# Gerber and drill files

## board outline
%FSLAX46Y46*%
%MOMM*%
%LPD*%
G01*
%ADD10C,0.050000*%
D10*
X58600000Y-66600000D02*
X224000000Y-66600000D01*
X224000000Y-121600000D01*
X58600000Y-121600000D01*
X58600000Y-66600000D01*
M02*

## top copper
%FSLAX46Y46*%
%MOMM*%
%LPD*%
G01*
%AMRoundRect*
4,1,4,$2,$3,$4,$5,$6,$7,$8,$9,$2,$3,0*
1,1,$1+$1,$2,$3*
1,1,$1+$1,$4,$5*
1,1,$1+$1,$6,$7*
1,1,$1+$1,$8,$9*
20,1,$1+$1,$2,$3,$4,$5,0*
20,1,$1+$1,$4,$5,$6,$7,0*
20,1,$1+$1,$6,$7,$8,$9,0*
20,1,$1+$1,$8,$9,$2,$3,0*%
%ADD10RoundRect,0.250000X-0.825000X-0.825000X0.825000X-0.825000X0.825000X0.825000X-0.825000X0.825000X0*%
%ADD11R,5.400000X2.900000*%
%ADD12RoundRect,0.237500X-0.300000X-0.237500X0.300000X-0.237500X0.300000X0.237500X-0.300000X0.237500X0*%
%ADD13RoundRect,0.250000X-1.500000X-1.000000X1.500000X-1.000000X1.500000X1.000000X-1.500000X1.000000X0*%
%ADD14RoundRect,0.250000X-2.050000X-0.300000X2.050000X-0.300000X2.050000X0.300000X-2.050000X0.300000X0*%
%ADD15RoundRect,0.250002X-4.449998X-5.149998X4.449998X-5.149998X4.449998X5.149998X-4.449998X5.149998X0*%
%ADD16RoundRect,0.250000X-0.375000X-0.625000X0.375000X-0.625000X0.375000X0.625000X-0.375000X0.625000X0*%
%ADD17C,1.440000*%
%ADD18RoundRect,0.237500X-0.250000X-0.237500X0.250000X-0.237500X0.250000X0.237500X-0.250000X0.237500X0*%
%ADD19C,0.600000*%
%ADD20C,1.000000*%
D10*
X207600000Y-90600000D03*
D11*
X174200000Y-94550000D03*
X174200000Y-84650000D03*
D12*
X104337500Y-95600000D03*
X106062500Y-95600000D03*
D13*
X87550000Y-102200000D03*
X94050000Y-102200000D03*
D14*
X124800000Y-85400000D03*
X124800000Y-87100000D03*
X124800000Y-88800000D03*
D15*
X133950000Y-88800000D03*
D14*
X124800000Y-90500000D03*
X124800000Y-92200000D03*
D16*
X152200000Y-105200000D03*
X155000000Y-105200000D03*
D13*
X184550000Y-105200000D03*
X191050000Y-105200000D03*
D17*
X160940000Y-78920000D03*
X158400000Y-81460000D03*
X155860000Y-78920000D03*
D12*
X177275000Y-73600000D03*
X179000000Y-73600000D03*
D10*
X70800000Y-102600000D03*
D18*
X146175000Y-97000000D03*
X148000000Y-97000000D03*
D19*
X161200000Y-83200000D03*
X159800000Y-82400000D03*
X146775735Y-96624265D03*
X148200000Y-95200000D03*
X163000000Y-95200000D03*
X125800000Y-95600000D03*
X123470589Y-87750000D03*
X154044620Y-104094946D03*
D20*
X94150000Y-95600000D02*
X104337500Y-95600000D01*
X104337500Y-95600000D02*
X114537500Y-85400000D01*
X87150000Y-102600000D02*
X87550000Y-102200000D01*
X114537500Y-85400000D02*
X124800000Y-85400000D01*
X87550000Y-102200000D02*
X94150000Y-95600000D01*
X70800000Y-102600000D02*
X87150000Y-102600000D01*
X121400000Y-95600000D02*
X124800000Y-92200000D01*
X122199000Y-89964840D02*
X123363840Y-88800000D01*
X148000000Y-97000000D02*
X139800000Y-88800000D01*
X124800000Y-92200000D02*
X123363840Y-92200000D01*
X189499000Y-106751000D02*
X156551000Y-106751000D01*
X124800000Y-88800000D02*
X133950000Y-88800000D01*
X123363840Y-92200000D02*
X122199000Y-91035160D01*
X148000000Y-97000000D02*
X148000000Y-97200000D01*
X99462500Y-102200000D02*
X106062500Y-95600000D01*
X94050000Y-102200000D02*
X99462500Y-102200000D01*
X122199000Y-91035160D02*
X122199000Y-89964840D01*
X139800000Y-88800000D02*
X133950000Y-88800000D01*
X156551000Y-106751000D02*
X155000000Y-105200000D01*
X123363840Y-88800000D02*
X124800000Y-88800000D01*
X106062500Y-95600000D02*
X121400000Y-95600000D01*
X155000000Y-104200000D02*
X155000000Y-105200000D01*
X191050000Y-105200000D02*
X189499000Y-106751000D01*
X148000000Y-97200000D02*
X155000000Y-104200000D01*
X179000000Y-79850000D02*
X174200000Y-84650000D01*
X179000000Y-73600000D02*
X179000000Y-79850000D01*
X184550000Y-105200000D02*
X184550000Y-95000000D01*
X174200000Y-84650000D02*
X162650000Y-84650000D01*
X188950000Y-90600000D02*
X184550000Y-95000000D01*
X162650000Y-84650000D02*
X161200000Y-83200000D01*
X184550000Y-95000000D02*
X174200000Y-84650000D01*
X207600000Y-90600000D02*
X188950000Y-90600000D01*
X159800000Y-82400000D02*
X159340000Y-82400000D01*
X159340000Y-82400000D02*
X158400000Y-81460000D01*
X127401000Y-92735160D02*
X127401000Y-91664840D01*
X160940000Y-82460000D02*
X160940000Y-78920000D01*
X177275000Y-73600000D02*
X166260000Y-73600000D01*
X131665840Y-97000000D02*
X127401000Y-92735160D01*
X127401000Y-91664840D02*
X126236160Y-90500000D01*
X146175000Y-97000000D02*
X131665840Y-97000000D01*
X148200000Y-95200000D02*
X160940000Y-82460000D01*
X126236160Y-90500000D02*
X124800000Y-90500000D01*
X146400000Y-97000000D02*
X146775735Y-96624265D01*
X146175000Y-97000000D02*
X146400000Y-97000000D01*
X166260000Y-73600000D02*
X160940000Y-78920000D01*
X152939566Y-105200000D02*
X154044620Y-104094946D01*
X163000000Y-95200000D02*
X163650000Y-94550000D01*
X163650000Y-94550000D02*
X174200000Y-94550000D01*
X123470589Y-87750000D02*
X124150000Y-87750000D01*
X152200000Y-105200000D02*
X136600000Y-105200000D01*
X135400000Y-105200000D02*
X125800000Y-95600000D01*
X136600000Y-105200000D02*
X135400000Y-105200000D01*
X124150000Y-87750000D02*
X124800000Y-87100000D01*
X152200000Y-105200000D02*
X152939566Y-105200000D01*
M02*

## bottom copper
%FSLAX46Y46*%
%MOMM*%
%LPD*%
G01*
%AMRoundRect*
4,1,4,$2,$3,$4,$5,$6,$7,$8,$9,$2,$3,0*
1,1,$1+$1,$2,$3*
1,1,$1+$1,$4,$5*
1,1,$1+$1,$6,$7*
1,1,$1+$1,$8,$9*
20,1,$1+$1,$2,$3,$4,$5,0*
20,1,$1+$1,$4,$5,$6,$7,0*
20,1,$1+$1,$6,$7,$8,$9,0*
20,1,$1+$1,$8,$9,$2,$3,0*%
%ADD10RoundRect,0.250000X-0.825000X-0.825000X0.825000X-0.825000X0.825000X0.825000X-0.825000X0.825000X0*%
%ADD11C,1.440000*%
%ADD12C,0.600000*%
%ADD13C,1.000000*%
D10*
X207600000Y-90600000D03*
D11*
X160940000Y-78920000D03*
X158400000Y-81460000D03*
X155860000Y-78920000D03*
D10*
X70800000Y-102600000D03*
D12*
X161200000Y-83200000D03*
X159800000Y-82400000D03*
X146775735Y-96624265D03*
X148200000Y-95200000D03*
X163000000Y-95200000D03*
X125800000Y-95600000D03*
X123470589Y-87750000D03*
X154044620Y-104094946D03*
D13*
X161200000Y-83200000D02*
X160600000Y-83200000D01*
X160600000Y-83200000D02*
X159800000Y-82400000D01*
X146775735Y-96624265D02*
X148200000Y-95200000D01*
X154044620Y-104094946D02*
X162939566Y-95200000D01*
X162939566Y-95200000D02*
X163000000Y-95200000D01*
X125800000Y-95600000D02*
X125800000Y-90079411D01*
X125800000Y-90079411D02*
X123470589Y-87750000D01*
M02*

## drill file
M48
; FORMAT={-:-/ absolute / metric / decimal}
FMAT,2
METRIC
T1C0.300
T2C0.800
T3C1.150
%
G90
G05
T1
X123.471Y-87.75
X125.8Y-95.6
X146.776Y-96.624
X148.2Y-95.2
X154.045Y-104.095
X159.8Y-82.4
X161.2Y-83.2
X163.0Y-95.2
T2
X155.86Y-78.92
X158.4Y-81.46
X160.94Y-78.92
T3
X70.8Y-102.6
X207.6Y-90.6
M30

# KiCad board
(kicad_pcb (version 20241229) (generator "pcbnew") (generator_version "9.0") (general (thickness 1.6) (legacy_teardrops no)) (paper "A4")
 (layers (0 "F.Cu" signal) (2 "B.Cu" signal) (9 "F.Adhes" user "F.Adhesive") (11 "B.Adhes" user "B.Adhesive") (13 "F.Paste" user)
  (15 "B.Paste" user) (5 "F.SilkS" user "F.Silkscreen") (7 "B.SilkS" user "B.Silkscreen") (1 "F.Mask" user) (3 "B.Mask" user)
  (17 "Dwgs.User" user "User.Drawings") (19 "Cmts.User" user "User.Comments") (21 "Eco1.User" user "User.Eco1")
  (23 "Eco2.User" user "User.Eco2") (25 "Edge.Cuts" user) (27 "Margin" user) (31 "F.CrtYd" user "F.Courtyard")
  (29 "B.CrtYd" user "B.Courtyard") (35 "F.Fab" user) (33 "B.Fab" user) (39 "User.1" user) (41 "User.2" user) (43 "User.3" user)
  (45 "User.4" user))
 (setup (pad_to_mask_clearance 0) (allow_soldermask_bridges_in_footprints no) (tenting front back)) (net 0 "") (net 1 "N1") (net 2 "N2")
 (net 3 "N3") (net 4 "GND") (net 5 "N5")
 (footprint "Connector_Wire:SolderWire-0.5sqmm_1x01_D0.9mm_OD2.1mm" (layer "F.Cu") (at 207.6 90.6)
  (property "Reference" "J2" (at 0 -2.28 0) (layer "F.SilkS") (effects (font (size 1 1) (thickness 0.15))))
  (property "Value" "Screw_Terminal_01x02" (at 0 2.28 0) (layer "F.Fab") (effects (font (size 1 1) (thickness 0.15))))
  (pad "1" thru_hole roundrect (at 0 0) (size 2.15 2.15) (drill 1.15) (layers "*.Cu" "*.Mask") (remove_unused_layers no)
   (roundrect_rratio 0.116279) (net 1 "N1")))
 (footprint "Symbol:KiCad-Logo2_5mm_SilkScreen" (layer "F.Cu") (at 66.4 70.6)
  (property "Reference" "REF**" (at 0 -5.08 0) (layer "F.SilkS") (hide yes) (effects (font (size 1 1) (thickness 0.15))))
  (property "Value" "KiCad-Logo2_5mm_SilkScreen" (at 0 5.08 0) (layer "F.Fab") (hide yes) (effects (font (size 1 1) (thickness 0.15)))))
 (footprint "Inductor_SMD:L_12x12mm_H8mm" (layer "F.Cu") (at 174.2 89.6 90)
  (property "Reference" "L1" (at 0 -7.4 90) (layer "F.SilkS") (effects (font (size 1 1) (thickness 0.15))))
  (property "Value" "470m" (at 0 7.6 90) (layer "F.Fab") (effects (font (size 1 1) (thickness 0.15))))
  (pad "1" smd rect (at -4.95 0 90) (size 2.9 5.4) (layers "F.Cu" "F.Mask" "F.Paste") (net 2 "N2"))
  (pad "2" smd rect (at 4.95 0 90) (size 2.9 5.4) (layers "F.Cu" "F.Mask" "F.Paste") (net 1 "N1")))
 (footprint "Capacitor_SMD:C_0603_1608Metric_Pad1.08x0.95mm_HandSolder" (layer "F.Cu") (at 105.2 95.6)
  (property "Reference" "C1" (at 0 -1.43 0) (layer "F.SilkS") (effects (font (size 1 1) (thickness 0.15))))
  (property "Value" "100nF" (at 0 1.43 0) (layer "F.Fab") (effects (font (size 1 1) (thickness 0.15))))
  (pad "1" smd roundrect (at -0.8625 0) (size 1.075 0.95) (layers "F.Cu" "F.Mask" "F.Paste") (roundrect_rratio 0.25) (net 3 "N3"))
  (pad "2" smd roundrect (at 0.8625 0) (size 1.075 0.95) (layers "F.Cu" "F.Mask" "F.Paste") (roundrect_rratio 0.25) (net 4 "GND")))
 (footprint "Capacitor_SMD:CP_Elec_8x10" (layer "F.Cu") (at 90.8 102.2)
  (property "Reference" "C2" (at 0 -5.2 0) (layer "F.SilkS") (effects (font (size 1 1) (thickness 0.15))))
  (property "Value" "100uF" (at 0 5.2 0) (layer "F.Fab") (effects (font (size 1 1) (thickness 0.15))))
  (pad "1" smd roundrect (at -3.25 0) (size 3.5 2.5) (layers "F.Cu" "F.Mask" "F.Paste") (roundrect_rratio 0.1) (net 3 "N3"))
  (pad "2" smd roundrect (at 3.25 0) (size 3.5 2.5) (layers "F.Cu" "F.Mask" "F.Paste") (roundrect_rratio 0.1) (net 4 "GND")))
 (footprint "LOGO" (layer "F.Cu") (at 217.6 114.8)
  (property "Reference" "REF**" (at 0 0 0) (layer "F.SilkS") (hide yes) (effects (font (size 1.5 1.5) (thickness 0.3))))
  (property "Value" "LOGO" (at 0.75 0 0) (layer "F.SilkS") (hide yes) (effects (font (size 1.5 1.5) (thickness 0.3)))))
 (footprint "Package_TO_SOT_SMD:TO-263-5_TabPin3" (layer "F.Cu") (at 132.45 88.8)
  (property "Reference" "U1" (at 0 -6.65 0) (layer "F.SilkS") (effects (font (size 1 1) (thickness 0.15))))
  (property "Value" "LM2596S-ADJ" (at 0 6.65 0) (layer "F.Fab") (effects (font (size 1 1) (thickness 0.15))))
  (pad "" smd roundrect (at -0.925 -2.775) (size 4.55 5.25) (layers "F.Paste") (roundrect_rratio 0.054945))
  (pad "" smd roundrect (at -0.925 2.775) (size 4.55 5.25) (layers "F.Paste") (roundrect_rratio 0.054945))
  (pad "" smd roundrect (at 3.925 -2.775) (size 4.55 5.25) (layers "F.Paste") (roundrect_rratio 0.054945))
  (pad "" smd roundrect (at 3.925 2.775) (size 4.55 5.25) (layers "F.Paste") (roundrect_rratio 0.054945))
  (pad "1" smd roundrect (at -7.65 -3.4) (size 4.6 1.1) (layers "F.Cu" "F.Mask" "F.Paste") (roundrect_rratio 0.227273) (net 3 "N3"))
  (pad "2" smd roundrect (at -7.65 -1.7) (size 4.6 1.1) (layers "F.Cu" "F.Mask" "F.Paste") (roundrect_rratio 0.227273) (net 2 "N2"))
  (pad "3" smd roundrect (at -7.65 0) (size 4.6 1.1) (layers "F.Cu" "F.Mask" "F.Paste") (roundrect_rratio 0.227273) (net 4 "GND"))
  (pad "3" smd roundrect (at 1.5 0) (size 9.4 10.8) (layers "F.Cu" "F.Mask") (roundrect_rratio 0.026596) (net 4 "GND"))
  (pad "4" smd roundrect (at -7.65 1.7) (size 4.6 1.1) (layers "F.Cu" "F.Mask" "F.Paste") (roundrect_rratio 0.227273) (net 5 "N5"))
  (pad "5" smd roundrect (at -7.65 3.4) (size 4.6 1.1) (layers "F.Cu" "F.Mask" "F.Paste") (roundrect_rratio 0.227273) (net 4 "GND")))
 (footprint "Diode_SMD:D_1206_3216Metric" (layer "F.Cu") (at 153.6 105.2)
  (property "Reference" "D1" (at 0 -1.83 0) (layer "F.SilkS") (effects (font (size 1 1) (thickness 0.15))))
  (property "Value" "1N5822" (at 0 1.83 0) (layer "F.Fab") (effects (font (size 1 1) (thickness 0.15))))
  (pad "1" smd roundrect (at -1.4 0) (size 1.25 1.75) (layers "F.Cu" "F.Mask" "F.Paste") (roundrect_rratio 0.2) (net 2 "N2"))
  (pad "2" smd roundrect (at 1.4 0) (size 1.25 1.75) (layers "F.Cu" "F.Mask" "F.Paste") (roundrect_rratio 0.2) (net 4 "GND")))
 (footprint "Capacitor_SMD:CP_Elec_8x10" (layer "F.Cu") (at 187.8 105.2)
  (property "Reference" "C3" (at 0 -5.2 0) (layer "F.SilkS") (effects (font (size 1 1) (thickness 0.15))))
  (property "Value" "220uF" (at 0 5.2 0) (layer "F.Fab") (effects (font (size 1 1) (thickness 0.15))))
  (pad "1" smd roundrect (at -3.25 0) (size 3.5 2.5) (layers "F.Cu" "F.Mask" "F.Paste") (roundrect_rratio 0.1) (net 1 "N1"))
  (pad "2" smd roundrect (at 3.25 0) (size 3.5 2.5) (layers "F.Cu" "F.Mask" "F.Paste") (roundrect_rratio 0.1) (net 4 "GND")))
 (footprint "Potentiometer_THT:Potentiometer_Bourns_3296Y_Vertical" (layer "F.Cu") (at 160.94 78.92)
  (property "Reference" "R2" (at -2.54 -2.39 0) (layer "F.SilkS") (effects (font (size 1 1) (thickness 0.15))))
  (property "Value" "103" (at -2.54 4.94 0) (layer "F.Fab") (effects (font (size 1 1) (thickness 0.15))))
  (pad "1" thru_hole circle (at 0 0) (size 1.44 1.44) (drill 0.8) (layers "*.Cu" "*.Mask") (remove_unused_layers no) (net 5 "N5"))
  (pad "2" thru_hole circle (at -2.54 2.54) (size 1.44 1.44) (drill 0.8) (layers "*.Cu" "*.Mask") (remove_unused_layers no) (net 1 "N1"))
  (pad "3" thru_hole circle (at -5.08 0) (size 1.44 1.44) (drill 0.8) (layers "*.Cu" "*.Mask") (remove_unused_layers no)))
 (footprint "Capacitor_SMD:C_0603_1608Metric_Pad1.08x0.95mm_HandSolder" (layer "F.Cu") (at 178.1375 73.6)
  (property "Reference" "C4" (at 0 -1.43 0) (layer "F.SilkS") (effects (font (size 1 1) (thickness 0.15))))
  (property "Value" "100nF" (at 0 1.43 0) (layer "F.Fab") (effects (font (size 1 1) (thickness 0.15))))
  (pad "1" smd roundrect (at -0.8625 0) (size 1.075 0.95) (layers "F.Cu" "F.Mask" "F.Paste") (roundrect_rratio 0.25) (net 5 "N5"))
  (pad "2" smd roundrect (at 0.8625 0) (size 1.075 0.95) (layers "F.Cu" "F.Mask" "F.Paste") (roundrect_rratio 0.25) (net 1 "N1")))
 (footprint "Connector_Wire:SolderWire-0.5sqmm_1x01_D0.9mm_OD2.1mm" (layer "F.Cu") (at 70.8 102.6)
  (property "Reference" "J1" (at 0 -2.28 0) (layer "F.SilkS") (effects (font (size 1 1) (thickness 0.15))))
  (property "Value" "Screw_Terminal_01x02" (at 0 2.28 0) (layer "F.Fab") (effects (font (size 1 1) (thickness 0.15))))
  (pad "1" thru_hole roundrect (at 0 0) (size 2.15 2.15) (drill 1.15) (layers "*.Cu" "*.Mask") (remove_unused_layers no)
   (roundrect_rratio 0.116279) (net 3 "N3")))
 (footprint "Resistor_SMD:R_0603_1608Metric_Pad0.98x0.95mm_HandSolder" (layer "F.Cu") (at 147.0875 97)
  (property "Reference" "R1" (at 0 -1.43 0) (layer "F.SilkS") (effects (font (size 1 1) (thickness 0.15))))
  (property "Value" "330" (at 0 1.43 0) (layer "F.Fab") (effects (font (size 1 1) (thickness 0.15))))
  (pad "1" smd roundrect (at -0.9125 0) (size 0.975 0.95) (layers "F.Cu" "F.Mask" "F.Paste") (roundrect_rratio 0.25) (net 5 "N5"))
  (pad "2" smd roundrect (at 0.9125 0) (size 0.975 0.95) (layers "F.Cu" "F.Mask" "F.Paste") (roundrect_rratio 0.25) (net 4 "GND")))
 (gr_rect (start 58.6 66.6) (end 224 121.6) (stroke (width 0.05) (type default)) (fill no) (layer "Edge.Cuts"))
 (segment (start 94.15 95.6) (end 104.3375 95.6) (width 1) (layers "F.Cu" "F.Mask") (solder_mask_margin 1) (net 3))
 (segment (start 104.3375 95.6) (end 114.5375 85.4) (width 1) (layers "F.Cu" "F.Mask") (solder_mask_margin 1) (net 3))
 (segment (start 87.15 102.6) (end 87.55 102.2) (width 1) (layer "F.Cu") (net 3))
 (segment (start 114.5375 85.4) (end 124.8 85.4) (width 1) (layers "F.Cu" "F.Mask") (solder_mask_margin 1) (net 3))
 (segment (start 87.55 102.2) (end 94.15 95.6) (width 1) (layers "F.Cu" "F.Mask") (solder_mask_margin 1) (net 3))
 (segment (start 70.8 102.6) (end 87.15 102.6) (width 1) (layers "F.Cu" "F.Mask") (solder_mask_margin 1) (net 3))
 (segment (start 121.4 95.6) (end 124.8 92.2) (width 1) (layers "F.Cu" "F.Mask") (solder_mask_margin 1) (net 4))
 (segment (start 122.199 89.96484) (end 123.36384 88.8) (width 1) (layers "F.Cu" "F.Mask") (solder_mask_margin 1) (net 4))
 (segment (start 148 97) (end 139.8 88.8) (width 1) (layers "F.Cu" "F.Mask") (solder_mask_margin 1) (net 4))
 (segment (start 124.8 92.2) (end 123.36384 92.2) (width 1) (layer "F.Cu") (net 4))
 (segment (start 189.499 106.751) (end 156.551 106.751) (width 1) (layers "F.Cu" "F.Mask") (solder_mask_margin 1) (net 4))
 (segment (start 124.8 88.8) (end 133.95 88.8) (width 1) (layers "F.Cu" "F.Mask") (solder_mask_margin 1) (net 4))
 (segment (start 123.36384 92.2) (end 122.199 91.03516) (width 1) (layers "F.Cu" "F.Mask") (solder_mask_margin 1) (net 4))
 (segment (start 148 97) (end 148 97.2) (width 1) (layer "F.Cu") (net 4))
 (segment (start 99.4625 102.2) (end 106.0625 95.6) (width 1) (layers "F.Cu" "F.Mask") (solder_mask_margin 1) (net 4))
 (segment (start 94.05 102.2) (end 99.4625 102.2) (width 1) (layers "F.Cu" "F.Mask") (solder_mask_margin 1) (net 4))
 (segment (start 122.199 91.03516) (end 122.199 89.96484) (width 1) (layers "F.Cu" "F.Mask") (solder_mask_margin 1) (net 4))
 (segment (start 139.8 88.8) (end 133.95 88.8) (width 1) (layers "F.Cu" "F.Mask") (solder_mask_margin 1) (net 4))
 (segment (start 156.551 106.751) (end 155 105.2) (width 1) (layers "F.Cu" "F.Mask") (solder_mask_margin 1) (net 4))
 (segment (start 123.36384 88.8) (end 124.8 88.8) (width 1) (layers "F.Cu" "F.Mask") (solder_mask_margin 1) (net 4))
 (segment (start 106.0625 95.6) (end 121.4 95.6) (width 1) (layers "F.Cu" "F.Mask") (solder_mask_margin 1) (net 4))
 (segment (start 155 104.2) (end 155 105.2) (width 1) (layer "F.Cu") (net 4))
 (segment (start 191.05 105.2) (end 189.499 106.751) (width 1) (layers "F.Cu" "F.Mask") (solder_mask_margin 1) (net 4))
 (segment (start 148 97.2) (end 155 104.2) (width 1) (layers "F.Cu" "F.Mask") (solder_mask_margin 1) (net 4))
 (segment (start 179 79.85) (end 174.2 84.65) (width 1) (layers "F.Cu" "F.Mask") (solder_mask_margin 1) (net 1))
 (segment (start 179 73.6) (end 179 79.85) (width 1) (layers "F.Cu" "F.Mask") (solder_mask_margin 1) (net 1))
 (segment (start 184.55 105.2) (end 184.55 95) (width 1) (layers "F.Cu" "F.Mask") (solder_mask_margin 1) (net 1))
 (segment (start 174.2 84.65) (end 162.65 84.65) (width 1) (layers "F.Cu" "F.Mask") (solder_mask_margin 1) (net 1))
 (segment (start 188.95 90.6) (end 184.55 95) (width 1) (layers "F.Cu" "F.Mask") (solder_mask_margin 1) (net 1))
 (segment (start 162.65 84.65) (end 161.2 83.2) (width 1) (layers "F.Cu" "F.Mask") (solder_mask_margin 1) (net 1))
 (segment (start 184.55 95) (end 174.2 84.65) (width 1) (layers "F.Cu" "F.Mask") (solder_mask_margin 1) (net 1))
 (segment (start 207.6 90.6) (end 188.95 90.6) (width 1) (layers "F.Cu" "F.Mask") (solder_mask_margin 1) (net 1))
 (segment (start 159.8 82.4) (end 159.34 82.4) (width 1) (layers "F.Cu" "F.Mask") (solder_mask_margin 1) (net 1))
 (segment (start 159.34 82.4) (end 158.4 81.46) (width 1) (layers "F.Cu" "F.Mask") (solder_mask_margin 1) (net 1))
 (via (at 161.2 83.2) (size 0.6) (drill 0.3) (layers "F.Cu" "B.Cu") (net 1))
 (via (at 159.8 82.4) (size 0.6) (drill 0.3) (layers "F.Cu" "B.Cu") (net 1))
 (segment (start 161.2 83.2) (end 160.6 83.2) (width 1) (layers "B.Cu" "B.Mask") (solder_mask_margin 1) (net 1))
 (segment (start 160.6 83.2) (end 159.8 82.4) (width 1) (layers "B.Cu" "B.Mask") (solder_mask_margin 1) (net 1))
 (segment (start 127.401 92.73516) (end 127.401 91.66484) (width 1) (layer "F.Cu") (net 5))
 (segment (start 160.94 82.46) (end 160.94 78.92) (width 1) (layers "F.Cu" "F.Mask") (solder_mask_margin 1) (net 5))
 (segment (start 177.275 73.6) (end 166.26 73.6) (width 1) (layers "F.Cu" "F.Mask") (solder_mask_margin 1) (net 5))
 (segment (start 131.66584 97) (end 127.401 92.73516) (width 1) (layers "F.Cu" "F.Mask") (solder_mask_margin 1) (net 5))
 (segment (start 127.401 91.66484) (end 126.23616 90.5) (width 1) (layer "F.Cu") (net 5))
 (segment (start 146.175 97) (end 131.66584 97) (width 1) (layers "F.Cu" "F.Mask") (solder_mask_margin 1) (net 5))
 (segment (start 148.2 95.2) (end 160.94 82.46) (width 1) (layers "F.Cu" "F.Mask") (solder_mask_margin 1) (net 5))
 (segment (start 126.23616 90.5) (end 124.8 90.5) (width 1) (layer "F.Cu") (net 5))
 (segment (start 146.4 97) (end 146.775735 96.624265) (width 1) (layer "F.Cu") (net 5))
 (segment (start 146.175 97) (end 146.4 97) (width 1) (layer "F.Cu") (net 5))
 (segment (start 166.26 73.6) (end 160.94 78.92) (width 1) (layers "F.Cu" "F.Mask") (solder_mask_margin 1) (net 5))
 (via (at 146.775735 96.624265) (size 0.6) (drill 0.3) (layers "F.Cu" "B.Cu") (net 5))
 (via (at 148.2 95.2) (size 0.6) (drill 0.3) (layers "F.Cu" "B.Cu") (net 5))
 (segment (start 146.775735 96.624265) (end 148.2 95.2) (width 1) (layers "B.Cu" "B.Mask") (solder_mask_margin 1) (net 5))
 (segment (start 152.939566 105.2) (end 154.04462 104.094946) (width 1) (layers "F.Cu" "F.Mask") (solder_mask_margin 1) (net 2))
 (segment (start 163 95.2) (end 163.65 94.55) (width 1) (layers "F.Cu" "F.Mask") (solder_mask_margin 1) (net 2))
 (segment (start 163.65 94.55) (end 174.2 94.55) (width 1) (layers "F.Cu" "F.Mask") (solder_mask_margin 1) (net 2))
 (segment (start 123.470589 87.75) (end 124.15 87.75) (width 1) (layer "F.Cu") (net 2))
 (segment (start 152.2 105.2) (end 136.6 105.2) (width 1) (layers "F.Cu" "F.Mask") (solder_mask_margin 1) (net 2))
 (segment (start 135.4 105.2) (end 125.8 95.6) (width 1) (layers "F.Cu" "F.Mask") (solder_mask_margin 1) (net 2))
 (segment (start 136.6 105.2) (end 135.4 105.2) (width 1) (layer "F.Cu") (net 2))
 (segment (start 124.15 87.75) (end 124.8 87.1) (width 1) (layer "F.Cu") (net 2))
 (segment (start 152.2 105.2) (end 152.939566 105.2) (width 1) (layers "F.Cu" "F.Mask") (solder_mask_margin 1) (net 2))
 (via (at 163 95.2) (size 0.6) (drill 0.3) (layers "F.Cu" "B.Cu") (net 2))
 (via (at 125.8 95.6) (size 0.6) (drill 0.3) (layers "F.Cu" "B.Cu") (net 2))
 (via (at 123.470589 87.75) (size 0.6) (drill 0.3) (layers "F.Cu" "B.Cu") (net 2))
 (via (at 154.04462 104.094946) (size 0.6) (drill 0.3) (layers "F.Cu" "B.Cu") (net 2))
 (segment (start 154.04462 104.094946) (end 162.939566 95.2) (width 1) (layers "B.Cu" "B.Mask") (solder_mask_margin 1) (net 2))
 (segment (start 162.939566 95.2) (end 163 95.2) (width 1) (layer "B.Cu") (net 2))
 (segment (start 125.8 95.6) (end 125.8 90.079411) (width 1) (layers "B.Cu" "B.Mask") (solder_mask_margin 1) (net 2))
 (segment (start 125.8 90.079411) (end 123.470589 87.75) (width 1) (layers "B.Cu" "B.Mask") (solder_mask_margin 1) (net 2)))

